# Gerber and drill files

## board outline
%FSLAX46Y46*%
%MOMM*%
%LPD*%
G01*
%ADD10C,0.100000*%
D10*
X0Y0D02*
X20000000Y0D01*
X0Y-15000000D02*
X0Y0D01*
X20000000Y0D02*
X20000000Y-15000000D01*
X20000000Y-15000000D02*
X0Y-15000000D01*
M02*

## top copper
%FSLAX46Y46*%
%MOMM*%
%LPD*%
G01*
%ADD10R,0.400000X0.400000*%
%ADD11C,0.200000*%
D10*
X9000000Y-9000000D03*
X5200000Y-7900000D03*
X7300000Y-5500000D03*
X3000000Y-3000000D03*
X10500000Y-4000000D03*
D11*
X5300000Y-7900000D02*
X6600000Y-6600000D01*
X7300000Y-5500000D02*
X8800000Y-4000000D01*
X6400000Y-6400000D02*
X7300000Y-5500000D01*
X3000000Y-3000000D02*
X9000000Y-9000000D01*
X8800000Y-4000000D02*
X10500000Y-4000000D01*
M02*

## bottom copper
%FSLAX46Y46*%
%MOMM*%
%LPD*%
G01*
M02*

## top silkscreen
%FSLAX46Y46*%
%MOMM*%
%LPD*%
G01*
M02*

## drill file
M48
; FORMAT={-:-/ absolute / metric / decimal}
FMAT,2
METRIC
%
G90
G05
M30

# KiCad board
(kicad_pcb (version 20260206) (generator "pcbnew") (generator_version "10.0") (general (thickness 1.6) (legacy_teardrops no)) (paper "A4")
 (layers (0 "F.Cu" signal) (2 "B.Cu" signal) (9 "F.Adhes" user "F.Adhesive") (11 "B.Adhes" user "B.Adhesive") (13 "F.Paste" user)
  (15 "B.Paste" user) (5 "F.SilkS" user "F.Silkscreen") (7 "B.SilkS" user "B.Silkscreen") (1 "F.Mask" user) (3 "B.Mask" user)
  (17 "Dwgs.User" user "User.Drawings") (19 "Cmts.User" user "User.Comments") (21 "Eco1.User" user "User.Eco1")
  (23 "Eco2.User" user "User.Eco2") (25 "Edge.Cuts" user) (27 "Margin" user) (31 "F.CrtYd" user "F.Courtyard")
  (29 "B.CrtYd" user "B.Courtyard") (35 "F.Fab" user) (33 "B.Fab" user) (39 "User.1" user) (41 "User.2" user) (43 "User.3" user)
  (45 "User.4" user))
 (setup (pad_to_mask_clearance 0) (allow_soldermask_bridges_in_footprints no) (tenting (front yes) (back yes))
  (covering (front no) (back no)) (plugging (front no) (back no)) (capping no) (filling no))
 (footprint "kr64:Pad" (layer "F.Cu") (at 9 9)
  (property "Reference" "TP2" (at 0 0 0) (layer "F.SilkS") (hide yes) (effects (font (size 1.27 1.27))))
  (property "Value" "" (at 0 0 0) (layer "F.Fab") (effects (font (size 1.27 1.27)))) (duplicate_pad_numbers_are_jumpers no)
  (pad "1" smd rect (at 0 0) (size 0.4 0.4) (layers "F.Cu" "F.Mask" "F.Paste") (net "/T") (thermal_bridge_angle 45)))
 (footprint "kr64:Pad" (layer "F.Cu") (at 5.2 7.9)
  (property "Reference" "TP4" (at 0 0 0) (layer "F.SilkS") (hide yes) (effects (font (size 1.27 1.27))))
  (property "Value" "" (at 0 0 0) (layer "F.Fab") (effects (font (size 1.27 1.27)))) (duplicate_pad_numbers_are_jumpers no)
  (pad "1" smd rect (at 0 0) (size 0.4 0.4) (layers "F.Cu" "F.Mask" "F.Paste") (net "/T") (thermal_bridge_angle 45)))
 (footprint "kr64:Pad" (layer "F.Cu") (at 7.3 5.5)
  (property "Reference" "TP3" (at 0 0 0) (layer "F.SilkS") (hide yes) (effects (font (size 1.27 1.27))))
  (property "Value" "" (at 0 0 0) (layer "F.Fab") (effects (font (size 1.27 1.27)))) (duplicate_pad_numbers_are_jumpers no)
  (pad "1" smd rect (at 0 0) (size 0.4 0.4) (layers "F.Cu" "F.Mask" "F.Paste") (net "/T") (thermal_bridge_angle 45)))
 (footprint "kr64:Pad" (layer "F.Cu") (at 3 3)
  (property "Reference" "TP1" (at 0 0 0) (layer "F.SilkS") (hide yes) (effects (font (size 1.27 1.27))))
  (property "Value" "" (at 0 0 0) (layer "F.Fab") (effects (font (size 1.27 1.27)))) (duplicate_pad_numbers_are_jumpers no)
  (pad "1" smd rect (at 0 0) (size 0.4 0.4) (layers "F.Cu" "F.Mask" "F.Paste") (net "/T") (thermal_bridge_angle 45)))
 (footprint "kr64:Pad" (layer "F.Cu") (at 10.5 4)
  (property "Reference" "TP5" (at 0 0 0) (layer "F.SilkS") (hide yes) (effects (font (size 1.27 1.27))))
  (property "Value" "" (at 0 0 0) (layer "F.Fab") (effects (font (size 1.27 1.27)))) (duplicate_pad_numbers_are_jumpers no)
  (pad "1" smd rect (at 0 0) (size 0.4 0.4) (layers "F.Cu" "F.Mask" "F.Paste") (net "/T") (thermal_bridge_angle 45)))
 (gr_line (start 0 0) (end 20 0) (stroke (width 0.1) (type default)) (layer "Edge.Cuts"))
 (gr_line (start 0 15) (end 0 0) (stroke (width 0.1) (type default)) (layer "Edge.Cuts"))
 (gr_line (start 20 0) (end 20 15) (stroke (width 0.1) (type default)) (layer "Edge.Cuts"))
 (gr_line (start 20 15) (end 0 15) (stroke (width 0.1) (type default)) (layer "Edge.Cuts"))
 (segment (start 5.3 7.9) (end 6.6 6.6) (width 0.2) (layer "F.Cu") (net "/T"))
 (segment (start 7.3 5.5) (end 8.8 4) (width 0.2) (layer "F.Cu") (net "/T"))
 (segment (start 6.4 6.4) (end 7.3 5.5) (width 0.2) (layer "F.Cu") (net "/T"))
 (segment (start 3 3) (end 9 9) (width 0.2) (layer "F.Cu") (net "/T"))
 (segment (start 8.8 4) (end 10.5 4) (width 0.2) (layer "F.Cu") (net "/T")))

